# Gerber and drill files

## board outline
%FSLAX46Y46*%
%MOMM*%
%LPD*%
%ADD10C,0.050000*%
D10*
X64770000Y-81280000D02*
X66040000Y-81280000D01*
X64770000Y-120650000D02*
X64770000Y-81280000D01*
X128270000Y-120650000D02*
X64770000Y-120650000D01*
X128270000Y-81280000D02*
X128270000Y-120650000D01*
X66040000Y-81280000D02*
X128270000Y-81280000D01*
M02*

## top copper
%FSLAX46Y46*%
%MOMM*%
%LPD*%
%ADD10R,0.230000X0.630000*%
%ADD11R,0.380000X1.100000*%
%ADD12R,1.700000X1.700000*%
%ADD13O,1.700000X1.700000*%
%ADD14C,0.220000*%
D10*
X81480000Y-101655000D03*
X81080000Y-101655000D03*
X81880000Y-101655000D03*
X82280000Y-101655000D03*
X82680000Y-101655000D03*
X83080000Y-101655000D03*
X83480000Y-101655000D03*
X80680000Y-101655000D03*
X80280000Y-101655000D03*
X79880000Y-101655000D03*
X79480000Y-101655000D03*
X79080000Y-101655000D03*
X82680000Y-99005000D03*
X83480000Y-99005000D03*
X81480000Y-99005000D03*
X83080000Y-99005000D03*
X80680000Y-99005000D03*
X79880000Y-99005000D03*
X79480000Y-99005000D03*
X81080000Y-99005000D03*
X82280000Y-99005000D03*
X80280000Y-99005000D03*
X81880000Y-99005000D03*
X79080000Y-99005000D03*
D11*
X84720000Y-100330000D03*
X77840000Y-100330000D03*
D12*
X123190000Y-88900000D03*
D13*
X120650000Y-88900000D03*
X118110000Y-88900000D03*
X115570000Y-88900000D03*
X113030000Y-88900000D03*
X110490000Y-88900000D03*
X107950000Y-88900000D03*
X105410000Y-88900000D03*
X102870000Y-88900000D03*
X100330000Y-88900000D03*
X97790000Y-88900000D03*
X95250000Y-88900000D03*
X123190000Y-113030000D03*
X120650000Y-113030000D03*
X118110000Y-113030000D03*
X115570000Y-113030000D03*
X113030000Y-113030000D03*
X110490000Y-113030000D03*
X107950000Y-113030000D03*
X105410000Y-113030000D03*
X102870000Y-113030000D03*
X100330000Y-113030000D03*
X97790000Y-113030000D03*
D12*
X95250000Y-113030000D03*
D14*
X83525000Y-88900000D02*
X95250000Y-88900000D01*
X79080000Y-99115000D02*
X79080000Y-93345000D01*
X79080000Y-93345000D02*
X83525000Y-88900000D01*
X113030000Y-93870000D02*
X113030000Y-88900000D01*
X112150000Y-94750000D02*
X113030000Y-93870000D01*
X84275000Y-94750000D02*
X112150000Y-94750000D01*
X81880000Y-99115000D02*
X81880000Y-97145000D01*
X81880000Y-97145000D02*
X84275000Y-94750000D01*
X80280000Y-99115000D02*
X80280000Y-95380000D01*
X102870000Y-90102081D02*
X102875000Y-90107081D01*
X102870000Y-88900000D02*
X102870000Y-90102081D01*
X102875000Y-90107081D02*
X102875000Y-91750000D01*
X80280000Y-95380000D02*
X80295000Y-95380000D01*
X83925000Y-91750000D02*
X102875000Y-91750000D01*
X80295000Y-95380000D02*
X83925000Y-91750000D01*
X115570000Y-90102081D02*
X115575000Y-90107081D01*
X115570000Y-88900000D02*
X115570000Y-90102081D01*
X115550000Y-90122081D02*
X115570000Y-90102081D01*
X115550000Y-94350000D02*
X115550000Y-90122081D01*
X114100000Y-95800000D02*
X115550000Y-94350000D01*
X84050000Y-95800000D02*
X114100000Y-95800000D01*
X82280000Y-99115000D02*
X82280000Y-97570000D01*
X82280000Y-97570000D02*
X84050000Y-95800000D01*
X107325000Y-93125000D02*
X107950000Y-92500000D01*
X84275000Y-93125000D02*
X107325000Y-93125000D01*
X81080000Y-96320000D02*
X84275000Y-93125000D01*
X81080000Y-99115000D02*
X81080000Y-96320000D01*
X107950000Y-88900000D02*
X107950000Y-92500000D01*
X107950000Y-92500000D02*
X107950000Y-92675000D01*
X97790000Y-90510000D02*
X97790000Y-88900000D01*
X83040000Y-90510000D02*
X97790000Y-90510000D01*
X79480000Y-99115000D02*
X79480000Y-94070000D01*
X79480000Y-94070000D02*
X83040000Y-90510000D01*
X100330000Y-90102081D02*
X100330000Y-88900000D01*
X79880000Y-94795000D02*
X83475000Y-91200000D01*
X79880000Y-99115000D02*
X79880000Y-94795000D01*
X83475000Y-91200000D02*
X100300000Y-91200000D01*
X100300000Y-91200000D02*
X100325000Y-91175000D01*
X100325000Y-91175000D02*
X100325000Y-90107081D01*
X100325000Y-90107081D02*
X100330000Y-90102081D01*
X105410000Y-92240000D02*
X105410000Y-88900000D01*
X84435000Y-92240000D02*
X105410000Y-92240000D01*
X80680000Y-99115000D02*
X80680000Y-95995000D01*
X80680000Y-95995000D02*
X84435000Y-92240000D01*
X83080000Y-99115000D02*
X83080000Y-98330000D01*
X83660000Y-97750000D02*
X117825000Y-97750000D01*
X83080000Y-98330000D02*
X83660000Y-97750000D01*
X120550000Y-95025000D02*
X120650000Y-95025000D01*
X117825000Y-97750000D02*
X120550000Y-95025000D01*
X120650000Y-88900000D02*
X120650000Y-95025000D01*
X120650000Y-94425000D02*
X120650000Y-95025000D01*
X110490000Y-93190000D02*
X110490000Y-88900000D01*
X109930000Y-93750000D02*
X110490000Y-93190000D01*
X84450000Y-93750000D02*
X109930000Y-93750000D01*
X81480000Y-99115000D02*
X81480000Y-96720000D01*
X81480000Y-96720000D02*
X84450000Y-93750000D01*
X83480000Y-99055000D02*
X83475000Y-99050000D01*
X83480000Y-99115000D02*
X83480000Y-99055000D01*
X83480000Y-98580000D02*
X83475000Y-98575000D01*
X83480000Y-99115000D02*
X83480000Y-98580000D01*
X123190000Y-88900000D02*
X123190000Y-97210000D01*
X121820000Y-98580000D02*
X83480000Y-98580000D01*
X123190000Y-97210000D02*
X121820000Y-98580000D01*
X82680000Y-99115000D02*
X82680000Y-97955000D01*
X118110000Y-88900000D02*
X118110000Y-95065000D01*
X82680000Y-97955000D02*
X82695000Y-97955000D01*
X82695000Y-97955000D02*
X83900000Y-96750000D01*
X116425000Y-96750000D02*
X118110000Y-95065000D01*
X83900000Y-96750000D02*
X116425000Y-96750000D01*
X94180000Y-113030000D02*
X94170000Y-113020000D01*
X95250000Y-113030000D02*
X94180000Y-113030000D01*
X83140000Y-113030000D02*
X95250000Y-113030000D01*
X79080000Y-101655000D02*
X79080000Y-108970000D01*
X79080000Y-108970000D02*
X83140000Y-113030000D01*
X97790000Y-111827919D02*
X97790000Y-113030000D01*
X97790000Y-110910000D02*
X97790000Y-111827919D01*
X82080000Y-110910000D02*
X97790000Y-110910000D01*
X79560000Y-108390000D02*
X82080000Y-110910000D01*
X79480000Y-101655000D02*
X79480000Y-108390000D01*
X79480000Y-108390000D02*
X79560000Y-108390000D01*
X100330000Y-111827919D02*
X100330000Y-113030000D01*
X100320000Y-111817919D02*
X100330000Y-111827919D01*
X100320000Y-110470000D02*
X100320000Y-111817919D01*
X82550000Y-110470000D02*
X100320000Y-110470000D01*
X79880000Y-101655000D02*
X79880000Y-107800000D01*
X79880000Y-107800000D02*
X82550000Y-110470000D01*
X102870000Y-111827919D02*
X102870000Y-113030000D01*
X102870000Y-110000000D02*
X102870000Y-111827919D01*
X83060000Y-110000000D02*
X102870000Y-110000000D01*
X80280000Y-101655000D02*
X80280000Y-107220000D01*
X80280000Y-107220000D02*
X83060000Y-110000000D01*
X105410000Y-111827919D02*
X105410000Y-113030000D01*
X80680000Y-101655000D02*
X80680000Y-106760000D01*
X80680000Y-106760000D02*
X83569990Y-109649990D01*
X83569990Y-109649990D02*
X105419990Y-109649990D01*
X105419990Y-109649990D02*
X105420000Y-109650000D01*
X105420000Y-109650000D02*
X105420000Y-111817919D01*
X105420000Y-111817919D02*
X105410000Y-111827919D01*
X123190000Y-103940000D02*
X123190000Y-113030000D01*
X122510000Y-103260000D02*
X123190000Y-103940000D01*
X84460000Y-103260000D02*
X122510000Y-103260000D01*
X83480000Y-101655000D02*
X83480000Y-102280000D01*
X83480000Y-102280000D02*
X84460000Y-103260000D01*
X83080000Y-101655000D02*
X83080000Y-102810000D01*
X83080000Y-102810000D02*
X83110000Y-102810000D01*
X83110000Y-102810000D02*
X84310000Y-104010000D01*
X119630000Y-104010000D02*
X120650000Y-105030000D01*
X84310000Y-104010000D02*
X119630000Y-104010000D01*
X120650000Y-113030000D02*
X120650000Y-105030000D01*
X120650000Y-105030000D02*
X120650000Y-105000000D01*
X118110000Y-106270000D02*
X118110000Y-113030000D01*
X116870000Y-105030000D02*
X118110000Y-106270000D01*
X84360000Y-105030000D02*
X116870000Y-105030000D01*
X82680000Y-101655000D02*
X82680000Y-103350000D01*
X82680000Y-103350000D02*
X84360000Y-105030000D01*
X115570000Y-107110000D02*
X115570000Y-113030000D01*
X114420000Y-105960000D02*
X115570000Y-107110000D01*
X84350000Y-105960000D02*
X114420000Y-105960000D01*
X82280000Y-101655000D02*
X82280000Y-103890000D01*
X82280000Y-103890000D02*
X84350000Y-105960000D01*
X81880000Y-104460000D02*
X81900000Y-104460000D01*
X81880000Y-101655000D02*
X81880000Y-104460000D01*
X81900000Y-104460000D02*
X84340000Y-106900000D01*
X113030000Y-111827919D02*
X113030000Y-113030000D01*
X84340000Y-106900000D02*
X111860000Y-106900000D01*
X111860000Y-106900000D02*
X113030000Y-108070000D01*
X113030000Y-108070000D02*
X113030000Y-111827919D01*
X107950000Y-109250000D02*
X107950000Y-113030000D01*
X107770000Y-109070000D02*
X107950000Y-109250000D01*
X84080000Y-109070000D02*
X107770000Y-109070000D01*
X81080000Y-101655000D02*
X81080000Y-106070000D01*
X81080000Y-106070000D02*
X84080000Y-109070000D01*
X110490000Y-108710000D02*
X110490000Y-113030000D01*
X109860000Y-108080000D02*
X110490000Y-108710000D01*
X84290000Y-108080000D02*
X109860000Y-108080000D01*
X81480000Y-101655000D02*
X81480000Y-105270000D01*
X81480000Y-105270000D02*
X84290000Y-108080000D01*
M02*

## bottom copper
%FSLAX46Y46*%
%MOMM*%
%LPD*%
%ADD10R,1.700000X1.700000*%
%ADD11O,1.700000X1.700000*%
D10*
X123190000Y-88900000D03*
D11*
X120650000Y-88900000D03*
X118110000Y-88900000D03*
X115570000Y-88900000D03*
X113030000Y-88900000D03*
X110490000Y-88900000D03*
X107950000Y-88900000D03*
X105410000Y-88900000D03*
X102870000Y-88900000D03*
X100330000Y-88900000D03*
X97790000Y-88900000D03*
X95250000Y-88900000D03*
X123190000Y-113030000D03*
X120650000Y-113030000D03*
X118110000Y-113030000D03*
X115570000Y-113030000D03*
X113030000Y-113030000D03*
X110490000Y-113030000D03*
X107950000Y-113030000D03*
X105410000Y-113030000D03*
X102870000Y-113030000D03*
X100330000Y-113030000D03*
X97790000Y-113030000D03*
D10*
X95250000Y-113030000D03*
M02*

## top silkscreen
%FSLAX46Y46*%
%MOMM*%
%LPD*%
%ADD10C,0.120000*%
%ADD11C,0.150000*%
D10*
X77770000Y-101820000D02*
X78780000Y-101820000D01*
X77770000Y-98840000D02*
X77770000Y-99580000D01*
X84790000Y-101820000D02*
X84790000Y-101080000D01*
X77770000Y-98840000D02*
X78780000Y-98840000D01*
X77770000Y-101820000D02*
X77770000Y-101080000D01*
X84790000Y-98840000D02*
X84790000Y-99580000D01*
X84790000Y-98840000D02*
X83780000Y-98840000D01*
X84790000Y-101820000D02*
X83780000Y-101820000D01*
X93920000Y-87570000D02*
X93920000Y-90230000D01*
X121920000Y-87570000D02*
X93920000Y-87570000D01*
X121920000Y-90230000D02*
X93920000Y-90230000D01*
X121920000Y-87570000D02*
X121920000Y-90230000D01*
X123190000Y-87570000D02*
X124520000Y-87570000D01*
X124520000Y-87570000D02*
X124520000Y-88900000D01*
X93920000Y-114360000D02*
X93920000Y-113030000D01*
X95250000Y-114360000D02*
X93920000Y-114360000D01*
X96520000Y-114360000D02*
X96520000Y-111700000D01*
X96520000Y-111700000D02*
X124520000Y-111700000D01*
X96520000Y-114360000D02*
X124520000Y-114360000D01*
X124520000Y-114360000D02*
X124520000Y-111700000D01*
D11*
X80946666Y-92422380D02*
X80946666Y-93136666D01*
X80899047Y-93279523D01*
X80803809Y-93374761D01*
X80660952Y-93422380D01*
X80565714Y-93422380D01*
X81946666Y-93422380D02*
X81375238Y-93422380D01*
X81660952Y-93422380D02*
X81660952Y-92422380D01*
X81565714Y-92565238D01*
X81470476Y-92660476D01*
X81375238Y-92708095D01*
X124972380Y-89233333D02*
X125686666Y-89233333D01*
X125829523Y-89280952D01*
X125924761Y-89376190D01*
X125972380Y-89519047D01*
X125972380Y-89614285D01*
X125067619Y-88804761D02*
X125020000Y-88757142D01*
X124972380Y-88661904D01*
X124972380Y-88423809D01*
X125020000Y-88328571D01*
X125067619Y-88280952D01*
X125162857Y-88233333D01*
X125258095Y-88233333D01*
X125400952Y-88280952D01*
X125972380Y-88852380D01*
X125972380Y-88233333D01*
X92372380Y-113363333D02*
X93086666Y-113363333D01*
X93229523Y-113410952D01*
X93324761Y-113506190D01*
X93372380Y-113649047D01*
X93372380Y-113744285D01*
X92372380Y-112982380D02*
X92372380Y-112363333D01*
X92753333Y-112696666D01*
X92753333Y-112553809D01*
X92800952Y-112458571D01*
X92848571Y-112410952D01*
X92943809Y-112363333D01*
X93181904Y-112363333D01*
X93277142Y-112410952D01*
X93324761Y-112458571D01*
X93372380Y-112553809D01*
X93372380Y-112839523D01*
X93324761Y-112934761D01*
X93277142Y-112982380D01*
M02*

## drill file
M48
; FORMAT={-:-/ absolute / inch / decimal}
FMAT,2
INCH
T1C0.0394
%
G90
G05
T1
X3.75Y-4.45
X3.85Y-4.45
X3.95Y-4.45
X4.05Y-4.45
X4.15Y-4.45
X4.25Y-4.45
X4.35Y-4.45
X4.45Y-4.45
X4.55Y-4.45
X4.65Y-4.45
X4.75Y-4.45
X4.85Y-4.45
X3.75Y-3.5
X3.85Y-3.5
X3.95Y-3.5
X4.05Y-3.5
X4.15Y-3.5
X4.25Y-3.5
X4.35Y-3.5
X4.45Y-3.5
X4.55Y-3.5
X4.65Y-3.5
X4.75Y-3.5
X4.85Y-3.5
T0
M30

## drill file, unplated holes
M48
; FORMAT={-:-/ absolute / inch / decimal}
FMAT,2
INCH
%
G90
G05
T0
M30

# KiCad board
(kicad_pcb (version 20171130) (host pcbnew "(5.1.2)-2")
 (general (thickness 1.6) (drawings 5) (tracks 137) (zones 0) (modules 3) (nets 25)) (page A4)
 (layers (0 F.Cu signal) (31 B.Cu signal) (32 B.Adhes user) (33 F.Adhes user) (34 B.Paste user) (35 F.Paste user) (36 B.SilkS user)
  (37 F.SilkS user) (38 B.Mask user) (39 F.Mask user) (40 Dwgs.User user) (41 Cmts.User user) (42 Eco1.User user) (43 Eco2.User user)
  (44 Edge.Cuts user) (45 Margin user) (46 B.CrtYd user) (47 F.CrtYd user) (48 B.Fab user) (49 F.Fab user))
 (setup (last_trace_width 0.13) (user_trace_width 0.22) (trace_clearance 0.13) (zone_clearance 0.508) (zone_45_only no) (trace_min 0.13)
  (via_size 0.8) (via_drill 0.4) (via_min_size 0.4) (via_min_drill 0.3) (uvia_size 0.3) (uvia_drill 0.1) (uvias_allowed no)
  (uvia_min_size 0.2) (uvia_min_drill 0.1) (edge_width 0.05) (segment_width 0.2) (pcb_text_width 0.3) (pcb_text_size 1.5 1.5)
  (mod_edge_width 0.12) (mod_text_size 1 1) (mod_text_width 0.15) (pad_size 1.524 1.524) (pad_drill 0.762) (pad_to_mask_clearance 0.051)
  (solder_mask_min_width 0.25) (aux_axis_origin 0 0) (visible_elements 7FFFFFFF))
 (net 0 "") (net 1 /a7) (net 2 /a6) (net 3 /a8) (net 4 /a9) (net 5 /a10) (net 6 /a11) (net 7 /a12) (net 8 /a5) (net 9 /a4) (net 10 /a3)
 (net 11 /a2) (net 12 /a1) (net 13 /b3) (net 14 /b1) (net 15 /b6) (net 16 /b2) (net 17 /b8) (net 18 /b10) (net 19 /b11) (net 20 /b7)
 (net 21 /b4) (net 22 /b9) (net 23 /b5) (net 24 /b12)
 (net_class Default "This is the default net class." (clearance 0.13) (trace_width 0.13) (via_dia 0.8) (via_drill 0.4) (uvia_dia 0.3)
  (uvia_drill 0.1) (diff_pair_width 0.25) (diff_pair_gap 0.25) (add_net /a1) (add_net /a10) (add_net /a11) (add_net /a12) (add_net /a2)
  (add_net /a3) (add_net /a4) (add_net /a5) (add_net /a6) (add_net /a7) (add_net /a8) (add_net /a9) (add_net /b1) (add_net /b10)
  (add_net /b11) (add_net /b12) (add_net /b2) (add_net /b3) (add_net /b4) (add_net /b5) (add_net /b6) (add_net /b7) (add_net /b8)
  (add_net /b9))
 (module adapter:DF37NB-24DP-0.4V (layer F.Cu) (at 81.28 100.33)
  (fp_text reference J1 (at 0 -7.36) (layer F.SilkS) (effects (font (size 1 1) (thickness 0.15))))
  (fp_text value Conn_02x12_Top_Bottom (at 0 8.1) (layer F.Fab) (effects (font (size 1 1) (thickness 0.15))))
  (fp_line (start -3.51 1.49) (end -2.5 1.49) (layer F.SilkS) (width 0.12))
  (fp_line (start -3.51 -1.49) (end -3.51 -0.75) (layer F.SilkS) (width 0.12))
  (fp_line (start 3.51 1.49) (end 3.51 0.75) (layer F.SilkS) (width 0.12))
  (fp_line (start -3.51 -1.49) (end -2.5 -1.49) (layer F.SilkS) (width 0.12))
  (fp_line (start -3.51 1.49) (end -3.51 0.75) (layer F.SilkS) (width 0.12))
  (fp_line (start 3.51 -1.49) (end 3.51 -0.75) (layer F.SilkS) (width 0.12))
  (fp_line (start 3.51 -1.49) (end 2.5 -1.49) (layer F.SilkS) (width 0.12))
  (fp_line (start 3.51 1.49) (end 2.5 1.49) (layer F.SilkS) (width 0.12))
  (pad 7 smd rect (at 0.2 1.325) (size 0.23 0.63) (layers F.Cu F.Paste F.Mask) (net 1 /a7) (solder_mask_margin 0.07))
  (pad 6 smd rect (at -0.2 1.325) (size 0.23 0.63) (layers F.Cu F.Paste F.Mask) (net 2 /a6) (solder_mask_margin 0.07))
  (pad 8 smd rect (at 0.6 1.325) (size 0.23 0.63) (layers F.Cu F.Paste F.Mask) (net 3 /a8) (solder_mask_margin 0.07))
  (pad 9 smd rect (at 1 1.325) (size 0.23 0.63) (layers F.Cu F.Paste F.Mask) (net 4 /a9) (solder_mask_margin 0.07))
  (pad 10 smd rect (at 1.4 1.325) (size 0.23 0.63) (layers F.Cu F.Paste F.Mask) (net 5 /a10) (solder_mask_margin 0.07))
  (pad 11 smd rect (at 1.8 1.325) (size 0.23 0.63) (layers F.Cu F.Paste F.Mask) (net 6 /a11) (solder_mask_margin 0.07))
  (pad 12 smd rect (at 2.2 1.325) (size 0.23 0.63) (layers F.Cu F.Paste F.Mask) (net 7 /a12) (solder_mask_margin 0.07))
  (pad 5 smd rect (at -0.6 1.325) (size 0.23 0.63) (layers F.Cu F.Paste F.Mask) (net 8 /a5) (solder_mask_margin 0.07))
  (pad 4 smd rect (at -1 1.325) (size 0.23 0.63) (layers F.Cu F.Paste F.Mask) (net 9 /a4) (solder_mask_margin 0.07))
  (pad 3 smd rect (at -1.4 1.325) (size 0.23 0.63) (layers F.Cu F.Paste F.Mask) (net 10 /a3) (solder_mask_margin 0.07))
  (pad 2 smd rect (at -1.8 1.325) (size 0.23 0.63) (layers F.Cu F.Paste F.Mask) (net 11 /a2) (solder_mask_margin 0.07))
  (pad 1 smd rect (at -2.2 1.325) (size 0.23 0.63) (layers F.Cu F.Paste F.Mask) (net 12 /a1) (solder_mask_margin 0.07))
  (pad 15 smd rect (at 1.4 -1.325) (size 0.23 0.63) (layers F.Cu F.Paste F.Mask) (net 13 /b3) (solder_mask_margin 0.07))
  (pad 13 smd rect (at 2.2 -1.325) (size 0.23 0.63) (layers F.Cu F.Paste F.Mask) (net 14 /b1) (solder_mask_margin 0.07))
  (pad 18 smd rect (at 0.2 -1.325) (size 0.23 0.63) (layers F.Cu F.Paste F.Mask) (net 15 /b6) (solder_mask_margin 0.07))
  (pad 14 smd rect (at 1.8 -1.325) (size 0.23 0.63) (layers F.Cu F.Paste F.Mask) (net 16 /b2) (solder_mask_margin 0.07))
  (pad 20 smd rect (at -0.6 -1.325) (size 0.23 0.63) (layers F.Cu F.Paste F.Mask) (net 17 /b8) (solder_mask_margin 0.07))
  (pad 22 smd rect (at -1.4 -1.325) (size 0.23 0.63) (layers F.Cu F.Paste F.Mask) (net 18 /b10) (solder_mask_margin 0.07))
  (pad 23 smd rect (at -1.8 -1.325) (size 0.23 0.63) (layers F.Cu F.Paste F.Mask) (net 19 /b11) (solder_mask_margin 0.07))
  (pad 19 smd rect (at -0.2 -1.325) (size 0.23 0.63) (layers F.Cu F.Paste F.Mask) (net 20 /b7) (solder_mask_margin 0.07))
  (pad 16 smd rect (at 1 -1.325) (size 0.23 0.63) (layers F.Cu F.Paste F.Mask) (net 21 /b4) (solder_mask_margin 0.07))
  (pad 21 smd rect (at -1 -1.325) (size 0.23 0.63) (layers F.Cu F.Paste F.Mask) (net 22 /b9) (solder_mask_margin 0.07))
  (pad 17 smd rect (at 0.6 -1.325) (size 0.23 0.63) (layers F.Cu F.Paste F.Mask) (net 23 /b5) (solder_mask_margin 0.07))
  (pad 24 smd rect (at -2.2 -1.325) (size 0.23 0.63) (layers F.Cu F.Paste F.Mask) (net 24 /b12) (solder_mask_margin 0.07))
  (pad "" smd rect (at 3.44 0) (size 0.38 1.1) (layers F.Cu F.Paste F.Mask) (solder_mask_margin 0.07))
  (pad "" smd rect (at -3.44 0) (size 0.38 1.1) (layers F.Cu F.Paste F.Mask) (solder_mask_margin 0.07)))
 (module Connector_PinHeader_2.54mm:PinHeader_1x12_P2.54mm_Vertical (layer F.Cu) (at 123.19 88.9 270)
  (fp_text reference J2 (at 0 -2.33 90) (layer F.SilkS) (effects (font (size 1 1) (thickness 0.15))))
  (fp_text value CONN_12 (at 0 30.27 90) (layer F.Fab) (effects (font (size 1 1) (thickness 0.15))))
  (fp_line (start -1.33 29.27) (end 1.33 29.27) (layer F.SilkS) (width 0.12))
  (fp_line (start -1.33 1.27) (end -1.33 29.27) (layer F.SilkS) (width 0.12))
  (fp_line (start 1.33 1.27) (end 1.33 29.27) (layer F.SilkS) (width 0.12))
  (fp_line (start -1.33 1.27) (end 1.33 1.27) (layer F.SilkS) (width 0.12))
  (fp_line (start -1.33 0) (end -1.33 -1.33) (layer F.SilkS) (width 0.12))
  (fp_line (start -1.33 -1.33) (end 0 -1.33) (layer F.SilkS) (width 0.12))
  (pad 1 thru_hole rect (at 0 0 270) (size 1.7 1.7) (drill 1) (layers *.Cu *.Mask) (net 14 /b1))
  (pad 2 thru_hole oval (at 0 2.54 270) (size 1.7 1.7) (drill 1) (layers *.Cu *.Mask) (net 16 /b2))
  (pad 3 thru_hole oval (at 0 5.08 270) (size 1.7 1.7) (drill 1) (layers *.Cu *.Mask) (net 13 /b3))
  (pad 4 thru_hole oval (at 0 7.62 270) (size 1.7 1.7) (drill 1) (layers *.Cu *.Mask) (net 21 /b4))
  (pad 5 thru_hole oval (at 0 10.16 270) (size 1.7 1.7) (drill 1) (layers *.Cu *.Mask) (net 23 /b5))
  (pad 6 thru_hole oval (at 0 12.7 270) (size 1.7 1.7) (drill 1) (layers *.Cu *.Mask) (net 15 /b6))
  (pad 7 thru_hole oval (at 0 15.24 270) (size 1.7 1.7) (drill 1) (layers *.Cu *.Mask) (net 20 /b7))
  (pad 8 thru_hole oval (at 0 17.78 270) (size 1.7 1.7) (drill 1) (layers *.Cu *.Mask) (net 17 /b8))
  (pad 9 thru_hole oval (at 0 20.32 270) (size 1.7 1.7) (drill 1) (layers *.Cu *.Mask) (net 22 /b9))
  (pad 10 thru_hole oval (at 0 22.86 270) (size 1.7 1.7) (drill 1) (layers *.Cu *.Mask) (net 18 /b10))
  (pad 11 thru_hole oval (at 0 25.4 270) (size 1.7 1.7) (drill 1) (layers *.Cu *.Mask) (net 19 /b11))
  (pad 12 thru_hole oval (at 0 27.94 270) (size 1.7 1.7) (drill 1) (layers *.Cu *.Mask) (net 24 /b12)))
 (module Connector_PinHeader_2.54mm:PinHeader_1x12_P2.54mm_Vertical (layer F.Cu) (at 95.25 113.03 90)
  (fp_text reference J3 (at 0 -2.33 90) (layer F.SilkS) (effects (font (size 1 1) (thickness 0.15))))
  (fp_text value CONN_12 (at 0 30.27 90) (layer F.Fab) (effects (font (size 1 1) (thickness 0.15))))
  (fp_line (start -1.33 -1.33) (end 0 -1.33) (layer F.SilkS) (width 0.12))
  (fp_line (start -1.33 0) (end -1.33 -1.33) (layer F.SilkS) (width 0.12))
  (fp_line (start -1.33 1.27) (end 1.33 1.27) (layer F.SilkS) (width 0.12))
  (fp_line (start 1.33 1.27) (end 1.33 29.27) (layer F.SilkS) (width 0.12))
  (fp_line (start -1.33 1.27) (end -1.33 29.27) (layer F.SilkS) (width 0.12))
  (fp_line (start -1.33 29.27) (end 1.33 29.27) (layer F.SilkS) (width 0.12))
  (pad 12 thru_hole oval (at 0 27.94 90) (size 1.7 1.7) (drill 1) (layers *.Cu *.Mask) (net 7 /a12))
  (pad 11 thru_hole oval (at 0 25.4 90) (size 1.7 1.7) (drill 1) (layers *.Cu *.Mask) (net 6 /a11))
  (pad 10 thru_hole oval (at 0 22.86 90) (size 1.7 1.7) (drill 1) (layers *.Cu *.Mask) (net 5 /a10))
  (pad 9 thru_hole oval (at 0 20.32 90) (size 1.7 1.7) (drill 1) (layers *.Cu *.Mask) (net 4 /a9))
  (pad 8 thru_hole oval (at 0 17.78 90) (size 1.7 1.7) (drill 1) (layers *.Cu *.Mask) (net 3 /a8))
  (pad 7 thru_hole oval (at 0 15.24 90) (size 1.7 1.7) (drill 1) (layers *.Cu *.Mask) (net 1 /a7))
  (pad 6 thru_hole oval (at 0 12.7 90) (size 1.7 1.7) (drill 1) (layers *.Cu *.Mask) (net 2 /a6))
  (pad 5 thru_hole oval (at 0 10.16 90) (size 1.7 1.7) (drill 1) (layers *.Cu *.Mask) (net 8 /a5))
  (pad 4 thru_hole oval (at 0 7.62 90) (size 1.7 1.7) (drill 1) (layers *.Cu *.Mask) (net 9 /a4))
  (pad 3 thru_hole oval (at 0 5.08 90) (size 1.7 1.7) (drill 1) (layers *.Cu *.Mask) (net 10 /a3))
  (pad 2 thru_hole oval (at 0 2.54 90) (size 1.7 1.7) (drill 1) (layers *.Cu *.Mask) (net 11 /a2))
  (pad 1 thru_hole rect (at 0 0 90) (size 1.7 1.7) (drill 1) (layers *.Cu *.Mask) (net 12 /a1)))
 (gr_line (start 64.77 81.28) (end 66.04 81.28) (layer Edge.Cuts) (width 0.05))
 (gr_line (start 64.77 120.65) (end 64.77 81.28) (layer Edge.Cuts) (width 0.05))
 (gr_line (start 128.27 120.65) (end 64.77 120.65) (layer Edge.Cuts) (width 0.05))
 (gr_line (start 128.27 81.28) (end 128.27 120.65) (layer Edge.Cuts) (width 0.05))
 (gr_line (start 66.04 81.28) (end 128.27 81.28) (layer Edge.Cuts) (width 0.05))
 (segment (start 83.525 88.9) (end 95.25 88.9) (width 0.22) (layer F.Cu) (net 24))
 (segment (start 79.08 99.115) (end 79.08 93.345) (width 0.22) (layer F.Cu) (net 24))
 (segment (start 79.08 93.345) (end 83.525 88.9) (width 0.22) (layer F.Cu) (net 24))
 (segment (start 113.03 93.87) (end 113.03 88.9) (width 0.22) (layer F.Cu) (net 23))
 (segment (start 112.15 94.75) (end 113.03 93.87) (width 0.22) (layer F.Cu) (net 23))
 (segment (start 84.275 94.75) (end 112.15 94.75) (width 0.22) (layer F.Cu) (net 23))
 (segment (start 81.88 99.115) (end 81.88 97.145) (width 0.22) (layer F.Cu) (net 23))
 (segment (start 81.88 97.145) (end 84.275 94.75) (width 0.22) (layer F.Cu) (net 23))
 (segment (start 80.28 99.115) (end 80.28 95.38) (width 0.22) (layer F.Cu) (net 22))
 (segment (start 102.87 90.102081) (end 102.875 90.107081) (width 0.22) (layer F.Cu) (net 22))
 (segment (start 102.87 88.9) (end 102.87 90.102081) (width 0.22) (layer F.Cu) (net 22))
 (segment (start 102.875 90.107081) (end 102.875 91.75) (width 0.22) (layer F.Cu) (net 22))
 (segment (start 80.28 95.38) (end 80.295 95.38) (width 0.22) (layer F.Cu) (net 22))
 (segment (start 83.925 91.75) (end 102.875 91.75) (width 0.22) (layer F.Cu) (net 22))
 (segment (start 80.295 95.38) (end 83.925 91.75) (width 0.22) (layer F.Cu) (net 22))
 (segment (start 115.57 90.102081) (end 115.575 90.107081) (width 0.22) (layer F.Cu) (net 21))
 (segment (start 115.57 88.9) (end 115.57 90.102081) (width 0.22) (layer F.Cu) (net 21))
 (segment (start 115.55 90.122081) (end 115.57 90.102081) (width 0.22) (layer F.Cu) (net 21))
 (segment (start 115.55 94.35) (end 115.55 90.122081) (width 0.22) (layer F.Cu) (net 21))
 (segment (start 114.1 95.8) (end 115.55 94.35) (width 0.22) (layer F.Cu) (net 21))
 (segment (start 84.05 95.8) (end 114.1 95.8) (width 0.22) (layer F.Cu) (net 21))
 (segment (start 82.28 99.115) (end 82.28 97.57) (width 0.22) (layer F.Cu) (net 21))
 (segment (start 82.28 97.57) (end 84.05 95.8) (width 0.22) (layer F.Cu) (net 21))
 (segment (start 107.325 93.125) (end 107.95 92.5) (width 0.22) (layer F.Cu) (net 20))
 (segment (start 84.275 93.125) (end 107.325 93.125) (width 0.22) (layer F.Cu) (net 20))
 (segment (start 81.08 96.32) (end 84.275 93.125) (width 0.22) (layer F.Cu) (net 20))
 (segment (start 81.08 99.115) (end 81.08 96.32) (width 0.22) (layer F.Cu) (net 20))
 (segment (start 107.95 88.9) (end 107.95 92.5) (width 0.22) (layer F.Cu) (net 20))
 (segment (start 107.95 92.5) (end 107.95 92.675) (width 0.22) (layer F.Cu) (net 20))
 (segment (start 97.79 90.51) (end 97.79 88.9) (width 0.22) (layer F.Cu) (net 19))
 (segment (start 83.04 90.51) (end 97.79 90.51) (width 0.22) (layer F.Cu) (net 19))
 (segment (start 79.48 99.115) (end 79.48 94.07) (width 0.22) (layer F.Cu) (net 19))
 (segment (start 79.48 94.07) (end 83.04 90.51) (width 0.22) (layer F.Cu) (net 19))
 (segment (start 100.33 90.102081) (end 100.33 88.9) (width 0.22) (layer F.Cu) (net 18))
 (segment (start 79.88 94.795) (end 83.475 91.2) (width 0.22) (layer F.Cu) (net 18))
 (segment (start 79.88 99.115) (end 79.88 94.795) (width 0.22) (layer F.Cu) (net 18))
 (segment (start 83.475 91.2) (end 100.3 91.2) (width 0.22) (layer F.Cu) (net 18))
 (segment (start 100.3 91.2) (end 100.325 91.175) (width 0.22) (layer F.Cu) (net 18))
 (segment (start 100.325 91.175) (end 100.325 90.107081) (width 0.22) (layer F.Cu) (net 18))
 (segment (start 100.325 90.107081) (end 100.33 90.102081) (width 0.22) (layer F.Cu) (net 18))
 (segment (start 105.41 92.24) (end 105.41 88.9) (width 0.22) (layer F.Cu) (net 17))
 (segment (start 84.435 92.24) (end 105.41 92.24) (width 0.22) (layer F.Cu) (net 17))
 (segment (start 80.68 99.115) (end 80.68 95.995) (width 0.22) (layer F.Cu) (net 17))
 (segment (start 80.68 95.995) (end 84.435 92.24) (width 0.22) (layer F.Cu) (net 17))
 (segment (start 83.08 99.115) (end 83.08 98.33) (width 0.22) (layer F.Cu) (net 16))
 (segment (start 83.66 97.75) (end 117.825 97.75) (width 0.22) (layer F.Cu) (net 16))
 (segment (start 83.08 98.33) (end 83.66 97.75) (width 0.22) (layer F.Cu) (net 16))
 (segment (start 120.55 95.025) (end 120.65 95.025) (width 0.22) (layer F.Cu) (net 16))
 (segment (start 117.825 97.75) (end 120.55 95.025) (width 0.22) (layer F.Cu) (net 16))
 (segment (start 120.65 88.9) (end 120.65 95.025) (width 0.22) (layer F.Cu) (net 16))
 (segment (start 120.65 94.425) (end 120.65 95.025) (width 0.22) (layer F.Cu) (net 16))
 (segment (start 110.49 93.19) (end 110.49 88.9) (width 0.22) (layer F.Cu) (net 15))
 (segment (start 109.93 93.75) (end 110.49 93.19) (width 0.22) (layer F.Cu) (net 15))
 (segment (start 84.45 93.75) (end 109.93 93.75) (width 0.22) (layer F.Cu) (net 15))
 (segment (start 81.48 99.115) (end 81.48 96.72) (width 0.22) (layer F.Cu) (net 15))
 (segment (start 81.48 96.72) (end 84.45 93.75) (width 0.22) (layer F.Cu) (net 15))
 (segment (start 83.48 99.055) (end 83.475 99.05) (width 0.22) (layer F.Cu) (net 14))
 (segment (start 83.48 99.115) (end 83.48 99.055) (width 0.22) (layer F.Cu) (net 14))
 (segment (start 83.48 98.58) (end 83.475 98.575) (width 0.22) (layer F.Cu) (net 14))
 (segment (start 83.48 99.115) (end 83.48 98.58) (width 0.22) (layer F.Cu) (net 14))
 (segment (start 123.19 88.9) (end 123.19 97.21) (width 0.22) (layer F.Cu) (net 14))
 (segment (start 121.82 98.58) (end 83.48 98.58) (width 0.22) (layer F.Cu) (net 14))
 (segment (start 123.19 97.21) (end 121.82 98.58) (width 0.22) (layer F.Cu) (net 14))
 (segment (start 82.68 99.115) (end 82.68 97.955) (width 0.22) (layer F.Cu) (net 13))
 (segment (start 118.11 88.9) (end 118.11 95.065) (width 0.22) (layer F.Cu) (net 13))
 (segment (start 82.68 97.955) (end 82.695 97.955) (width 0.22) (layer F.Cu) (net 13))
 (segment (start 82.695 97.955) (end 83.9 96.75) (width 0.22) (layer F.Cu) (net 13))
 (segment (start 116.425 96.75) (end 118.11 95.065) (width 0.22) (layer F.Cu) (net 13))
 (segment (start 83.9 96.75) (end 116.425 96.75) (width 0.22) (layer F.Cu) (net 13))
 (segment (start 94.18 113.03) (end 94.17 113.02) (width 0.22) (layer F.Cu) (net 12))
 (segment (start 95.25 113.03) (end 94.18 113.03) (width 0.22) (layer F.Cu) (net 12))
 (segment (start 83.14 113.03) (end 95.25 113.03) (width 0.22) (layer F.Cu) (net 12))
 (segment (start 79.08 101.655) (end 79.08 108.97) (width 0.22) (layer F.Cu) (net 12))
 (segment (start 79.08 108.97) (end 83.14 113.03) (width 0.22) (layer F.Cu) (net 12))
 (segment (start 97.79 111.827919) (end 97.79 113.03) (width 0.22) (layer F.Cu) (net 11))
 (segment (start 97.79 110.91) (end 97.79 111.827919) (width 0.22) (layer F.Cu) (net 11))
 (segment (start 82.08 110.91) (end 97.79 110.91) (width 0.22) (layer F.Cu) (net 11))
 (segment (start 79.56 108.39) (end 82.08 110.91) (width 0.22) (layer F.Cu) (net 11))
 (segment (start 79.48 101.655) (end 79.48 108.39) (width 0.22) (layer F.Cu) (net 11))
 (segment (start 79.48 108.39) (end 79.56 108.39) (width 0.22) (layer F.Cu) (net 11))
 (segment (start 100.33 111.827919) (end 100.33 113.03) (width 0.22) (layer F.Cu) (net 10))
 (segment (start 100.32 111.817919) (end 100.33 111.827919) (width 0.22) (layer F.Cu) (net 10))
 (segment (start 100.32 110.47) (end 100.32 111.817919) (width 0.22) (layer F.Cu) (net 10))
 (segment (start 82.55 110.47) (end 100.32 110.47) (width 0.22) (layer F.Cu) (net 10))
 (segment (start 79.88 101.655) (end 79.88 107.8) (width 0.22) (layer F.Cu) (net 10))
 (segment (start 79.88 107.8) (end 82.55 110.47) (width 0.22) (layer F.Cu) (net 10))
 (segment (start 102.87 111.827919) (end 102.87 113.03) (width 0.22) (layer F.Cu) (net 9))
 (segment (start 102.87 110) (end 102.87 111.827919) (width 0.22) (layer F.Cu) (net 9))
 (segment (start 83.06 110) (end 102.87 110) (width 0.22) (layer F.Cu) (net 9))
 (segment (start 80.28 101.655) (end 80.28 107.22) (width 0.22) (layer F.Cu) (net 9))
 (segment (start 80.28 107.22) (end 83.06 110) (width 0.22) (layer F.Cu) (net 9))
 (segment (start 105.41 111.827919) (end 105.41 113.03) (width 0.22) (layer F.Cu) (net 8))
 (segment (start 80.68 101.655) (end 80.68 106.76) (width 0.22) (layer F.Cu) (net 8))
 (segment (start 80.68 106.76) (end 83.56999 109.64999) (width 0.22) (layer F.Cu) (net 8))
 (segment (start 83.56999 109.64999) (end 105.41999 109.64999) (width 0.22) (layer F.Cu) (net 8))
 (segment (start 105.41999 109.64999) (end 105.42 109.65) (width 0.22) (layer F.Cu) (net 8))
 (segment (start 105.42 109.65) (end 105.42 111.817919) (width 0.22) (layer F.Cu) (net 8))
 (segment (start 105.42 111.817919) (end 105.41 111.827919) (width 0.22) (layer F.Cu) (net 8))
 (segment (start 123.19 103.94) (end 123.19 113.03) (width 0.22) (layer F.Cu) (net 7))
 (segment (start 122.51 103.26) (end 123.19 103.94) (width 0.22) (layer F.Cu) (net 7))
 (segment (start 84.46 103.26) (end 122.51 103.26) (width 0.22) (layer F.Cu) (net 7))
 (segment (start 83.48 101.655) (end 83.48 102.28) (width 0.22) (layer F.Cu) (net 7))
 (segment (start 83.48 102.28) (end 84.46 103.26) (width 0.22) (layer F.Cu) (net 7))
 (segment (start 83.08 101.655) (end 83.08 102.81) (width 0.22) (layer F.Cu) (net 6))
 (segment (start 83.08 102.81) (end 83.11 102.81) (width 0.22) (layer F.Cu) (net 6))
 (segment (start 83.11 102.81) (end 84.31 104.01) (width 0.22) (layer F.Cu) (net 6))
 (segment (start 119.63 104.01) (end 120.65 105.03) (width 0.22) (layer F.Cu) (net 6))
 (segment (start 84.31 104.01) (end 119.63 104.01) (width 0.22) (layer F.Cu) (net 6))
 (segment (start 120.65 113.03) (end 120.65 105.03) (width 0.22) (layer F.Cu) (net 6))
 (segment (start 120.65 105.03) (end 120.65 105) (width 0.22) (layer F.Cu) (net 6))
 (segment (start 118.11 106.27) (end 118.11 113.03) (width 0.22) (layer F.Cu) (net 5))
 (segment (start 116.87 105.03) (end 118.11 106.27) (width 0.22) (layer F.Cu) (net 5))
 (segment (start 84.36 105.03) (end 116.87 105.03) (width 0.22) (layer F.Cu) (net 5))
 (segment (start 82.68 101.655) (end 82.68 103.35) (width 0.22) (layer F.Cu) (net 5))
 (segment (start 82.68 103.35) (end 84.36 105.03) (width 0.22) (layer F.Cu) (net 5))
 (segment (start 115.57 107.11) (end 115.57 113.03) (width 0.22) (layer F.Cu) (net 4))
 (segment (start 114.42 105.96) (end 115.57 107.11) (width 0.22) (layer F.Cu) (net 4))
 (segment (start 84.35 105.96) (end 114.42 105.96) (width 0.22) (layer F.Cu) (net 4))
 (segment (start 82.28 101.655) (end 82.28 103.89) (width 0.22) (layer F.Cu) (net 4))
 (segment (start 82.28 103.89) (end 84.35 105.96) (width 0.22) (layer F.Cu) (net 4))
 (segment (start 81.88 104.46) (end 81.9 104.46) (width 0.22) (layer F.Cu) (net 3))
 (segment (start 81.88 101.655) (end 81.88 104.46) (width 0.22) (layer F.Cu) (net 3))
 (segment (start 81.9 104.46) (end 84.34 106.9) (width 0.22) (layer F.Cu) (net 3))
 (segment (start 113.03 111.827919) (end 113.03 113.03) (width 0.22) (layer F.Cu) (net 3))
 (segment (start 84.34 106.9) (end 111.86 106.9) (width 0.22) (layer F.Cu) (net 3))
 (segment (start 111.86 106.9) (end 113.03 108.07) (width 0.22) (layer F.Cu) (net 3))
 (segment (start 113.03 108.07) (end 113.03 111.827919) (width 0.22) (layer F.Cu) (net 3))
 (segment (start 107.95 109.25) (end 107.95 113.03) (width 0.22) (layer F.Cu) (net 2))
 (segment (start 107.77 109.07) (end 107.95 109.25) (width 0.22) (layer F.Cu) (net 2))
 (segment (start 84.08 109.07) (end 107.77 109.07) (width 0.22) (layer F.Cu) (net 2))
 (segment (start 81.08 101.655) (end 81.08 106.07) (width 0.22) (layer F.Cu) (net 2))
 (segment (start 81.08 106.07) (end 84.08 109.07) (width 0.22) (layer F.Cu) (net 2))
 (segment (start 110.49 108.71) (end 110.49 113.03) (width 0.22) (layer F.Cu) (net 1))
 (segment (start 109.86 108.08) (end 110.49 108.71) (width 0.22) (layer F.Cu) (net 1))
 (segment (start 84.29 108.08) (end 109.86 108.08) (width 0.22) (layer F.Cu) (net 1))
 (segment (start 81.48 101.655) (end 81.48 105.27) (width 0.22) (layer F.Cu) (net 1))
 (segment (start 81.48 105.27) (end 84.29 108.08) (width 0.22) (layer F.Cu) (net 1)))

